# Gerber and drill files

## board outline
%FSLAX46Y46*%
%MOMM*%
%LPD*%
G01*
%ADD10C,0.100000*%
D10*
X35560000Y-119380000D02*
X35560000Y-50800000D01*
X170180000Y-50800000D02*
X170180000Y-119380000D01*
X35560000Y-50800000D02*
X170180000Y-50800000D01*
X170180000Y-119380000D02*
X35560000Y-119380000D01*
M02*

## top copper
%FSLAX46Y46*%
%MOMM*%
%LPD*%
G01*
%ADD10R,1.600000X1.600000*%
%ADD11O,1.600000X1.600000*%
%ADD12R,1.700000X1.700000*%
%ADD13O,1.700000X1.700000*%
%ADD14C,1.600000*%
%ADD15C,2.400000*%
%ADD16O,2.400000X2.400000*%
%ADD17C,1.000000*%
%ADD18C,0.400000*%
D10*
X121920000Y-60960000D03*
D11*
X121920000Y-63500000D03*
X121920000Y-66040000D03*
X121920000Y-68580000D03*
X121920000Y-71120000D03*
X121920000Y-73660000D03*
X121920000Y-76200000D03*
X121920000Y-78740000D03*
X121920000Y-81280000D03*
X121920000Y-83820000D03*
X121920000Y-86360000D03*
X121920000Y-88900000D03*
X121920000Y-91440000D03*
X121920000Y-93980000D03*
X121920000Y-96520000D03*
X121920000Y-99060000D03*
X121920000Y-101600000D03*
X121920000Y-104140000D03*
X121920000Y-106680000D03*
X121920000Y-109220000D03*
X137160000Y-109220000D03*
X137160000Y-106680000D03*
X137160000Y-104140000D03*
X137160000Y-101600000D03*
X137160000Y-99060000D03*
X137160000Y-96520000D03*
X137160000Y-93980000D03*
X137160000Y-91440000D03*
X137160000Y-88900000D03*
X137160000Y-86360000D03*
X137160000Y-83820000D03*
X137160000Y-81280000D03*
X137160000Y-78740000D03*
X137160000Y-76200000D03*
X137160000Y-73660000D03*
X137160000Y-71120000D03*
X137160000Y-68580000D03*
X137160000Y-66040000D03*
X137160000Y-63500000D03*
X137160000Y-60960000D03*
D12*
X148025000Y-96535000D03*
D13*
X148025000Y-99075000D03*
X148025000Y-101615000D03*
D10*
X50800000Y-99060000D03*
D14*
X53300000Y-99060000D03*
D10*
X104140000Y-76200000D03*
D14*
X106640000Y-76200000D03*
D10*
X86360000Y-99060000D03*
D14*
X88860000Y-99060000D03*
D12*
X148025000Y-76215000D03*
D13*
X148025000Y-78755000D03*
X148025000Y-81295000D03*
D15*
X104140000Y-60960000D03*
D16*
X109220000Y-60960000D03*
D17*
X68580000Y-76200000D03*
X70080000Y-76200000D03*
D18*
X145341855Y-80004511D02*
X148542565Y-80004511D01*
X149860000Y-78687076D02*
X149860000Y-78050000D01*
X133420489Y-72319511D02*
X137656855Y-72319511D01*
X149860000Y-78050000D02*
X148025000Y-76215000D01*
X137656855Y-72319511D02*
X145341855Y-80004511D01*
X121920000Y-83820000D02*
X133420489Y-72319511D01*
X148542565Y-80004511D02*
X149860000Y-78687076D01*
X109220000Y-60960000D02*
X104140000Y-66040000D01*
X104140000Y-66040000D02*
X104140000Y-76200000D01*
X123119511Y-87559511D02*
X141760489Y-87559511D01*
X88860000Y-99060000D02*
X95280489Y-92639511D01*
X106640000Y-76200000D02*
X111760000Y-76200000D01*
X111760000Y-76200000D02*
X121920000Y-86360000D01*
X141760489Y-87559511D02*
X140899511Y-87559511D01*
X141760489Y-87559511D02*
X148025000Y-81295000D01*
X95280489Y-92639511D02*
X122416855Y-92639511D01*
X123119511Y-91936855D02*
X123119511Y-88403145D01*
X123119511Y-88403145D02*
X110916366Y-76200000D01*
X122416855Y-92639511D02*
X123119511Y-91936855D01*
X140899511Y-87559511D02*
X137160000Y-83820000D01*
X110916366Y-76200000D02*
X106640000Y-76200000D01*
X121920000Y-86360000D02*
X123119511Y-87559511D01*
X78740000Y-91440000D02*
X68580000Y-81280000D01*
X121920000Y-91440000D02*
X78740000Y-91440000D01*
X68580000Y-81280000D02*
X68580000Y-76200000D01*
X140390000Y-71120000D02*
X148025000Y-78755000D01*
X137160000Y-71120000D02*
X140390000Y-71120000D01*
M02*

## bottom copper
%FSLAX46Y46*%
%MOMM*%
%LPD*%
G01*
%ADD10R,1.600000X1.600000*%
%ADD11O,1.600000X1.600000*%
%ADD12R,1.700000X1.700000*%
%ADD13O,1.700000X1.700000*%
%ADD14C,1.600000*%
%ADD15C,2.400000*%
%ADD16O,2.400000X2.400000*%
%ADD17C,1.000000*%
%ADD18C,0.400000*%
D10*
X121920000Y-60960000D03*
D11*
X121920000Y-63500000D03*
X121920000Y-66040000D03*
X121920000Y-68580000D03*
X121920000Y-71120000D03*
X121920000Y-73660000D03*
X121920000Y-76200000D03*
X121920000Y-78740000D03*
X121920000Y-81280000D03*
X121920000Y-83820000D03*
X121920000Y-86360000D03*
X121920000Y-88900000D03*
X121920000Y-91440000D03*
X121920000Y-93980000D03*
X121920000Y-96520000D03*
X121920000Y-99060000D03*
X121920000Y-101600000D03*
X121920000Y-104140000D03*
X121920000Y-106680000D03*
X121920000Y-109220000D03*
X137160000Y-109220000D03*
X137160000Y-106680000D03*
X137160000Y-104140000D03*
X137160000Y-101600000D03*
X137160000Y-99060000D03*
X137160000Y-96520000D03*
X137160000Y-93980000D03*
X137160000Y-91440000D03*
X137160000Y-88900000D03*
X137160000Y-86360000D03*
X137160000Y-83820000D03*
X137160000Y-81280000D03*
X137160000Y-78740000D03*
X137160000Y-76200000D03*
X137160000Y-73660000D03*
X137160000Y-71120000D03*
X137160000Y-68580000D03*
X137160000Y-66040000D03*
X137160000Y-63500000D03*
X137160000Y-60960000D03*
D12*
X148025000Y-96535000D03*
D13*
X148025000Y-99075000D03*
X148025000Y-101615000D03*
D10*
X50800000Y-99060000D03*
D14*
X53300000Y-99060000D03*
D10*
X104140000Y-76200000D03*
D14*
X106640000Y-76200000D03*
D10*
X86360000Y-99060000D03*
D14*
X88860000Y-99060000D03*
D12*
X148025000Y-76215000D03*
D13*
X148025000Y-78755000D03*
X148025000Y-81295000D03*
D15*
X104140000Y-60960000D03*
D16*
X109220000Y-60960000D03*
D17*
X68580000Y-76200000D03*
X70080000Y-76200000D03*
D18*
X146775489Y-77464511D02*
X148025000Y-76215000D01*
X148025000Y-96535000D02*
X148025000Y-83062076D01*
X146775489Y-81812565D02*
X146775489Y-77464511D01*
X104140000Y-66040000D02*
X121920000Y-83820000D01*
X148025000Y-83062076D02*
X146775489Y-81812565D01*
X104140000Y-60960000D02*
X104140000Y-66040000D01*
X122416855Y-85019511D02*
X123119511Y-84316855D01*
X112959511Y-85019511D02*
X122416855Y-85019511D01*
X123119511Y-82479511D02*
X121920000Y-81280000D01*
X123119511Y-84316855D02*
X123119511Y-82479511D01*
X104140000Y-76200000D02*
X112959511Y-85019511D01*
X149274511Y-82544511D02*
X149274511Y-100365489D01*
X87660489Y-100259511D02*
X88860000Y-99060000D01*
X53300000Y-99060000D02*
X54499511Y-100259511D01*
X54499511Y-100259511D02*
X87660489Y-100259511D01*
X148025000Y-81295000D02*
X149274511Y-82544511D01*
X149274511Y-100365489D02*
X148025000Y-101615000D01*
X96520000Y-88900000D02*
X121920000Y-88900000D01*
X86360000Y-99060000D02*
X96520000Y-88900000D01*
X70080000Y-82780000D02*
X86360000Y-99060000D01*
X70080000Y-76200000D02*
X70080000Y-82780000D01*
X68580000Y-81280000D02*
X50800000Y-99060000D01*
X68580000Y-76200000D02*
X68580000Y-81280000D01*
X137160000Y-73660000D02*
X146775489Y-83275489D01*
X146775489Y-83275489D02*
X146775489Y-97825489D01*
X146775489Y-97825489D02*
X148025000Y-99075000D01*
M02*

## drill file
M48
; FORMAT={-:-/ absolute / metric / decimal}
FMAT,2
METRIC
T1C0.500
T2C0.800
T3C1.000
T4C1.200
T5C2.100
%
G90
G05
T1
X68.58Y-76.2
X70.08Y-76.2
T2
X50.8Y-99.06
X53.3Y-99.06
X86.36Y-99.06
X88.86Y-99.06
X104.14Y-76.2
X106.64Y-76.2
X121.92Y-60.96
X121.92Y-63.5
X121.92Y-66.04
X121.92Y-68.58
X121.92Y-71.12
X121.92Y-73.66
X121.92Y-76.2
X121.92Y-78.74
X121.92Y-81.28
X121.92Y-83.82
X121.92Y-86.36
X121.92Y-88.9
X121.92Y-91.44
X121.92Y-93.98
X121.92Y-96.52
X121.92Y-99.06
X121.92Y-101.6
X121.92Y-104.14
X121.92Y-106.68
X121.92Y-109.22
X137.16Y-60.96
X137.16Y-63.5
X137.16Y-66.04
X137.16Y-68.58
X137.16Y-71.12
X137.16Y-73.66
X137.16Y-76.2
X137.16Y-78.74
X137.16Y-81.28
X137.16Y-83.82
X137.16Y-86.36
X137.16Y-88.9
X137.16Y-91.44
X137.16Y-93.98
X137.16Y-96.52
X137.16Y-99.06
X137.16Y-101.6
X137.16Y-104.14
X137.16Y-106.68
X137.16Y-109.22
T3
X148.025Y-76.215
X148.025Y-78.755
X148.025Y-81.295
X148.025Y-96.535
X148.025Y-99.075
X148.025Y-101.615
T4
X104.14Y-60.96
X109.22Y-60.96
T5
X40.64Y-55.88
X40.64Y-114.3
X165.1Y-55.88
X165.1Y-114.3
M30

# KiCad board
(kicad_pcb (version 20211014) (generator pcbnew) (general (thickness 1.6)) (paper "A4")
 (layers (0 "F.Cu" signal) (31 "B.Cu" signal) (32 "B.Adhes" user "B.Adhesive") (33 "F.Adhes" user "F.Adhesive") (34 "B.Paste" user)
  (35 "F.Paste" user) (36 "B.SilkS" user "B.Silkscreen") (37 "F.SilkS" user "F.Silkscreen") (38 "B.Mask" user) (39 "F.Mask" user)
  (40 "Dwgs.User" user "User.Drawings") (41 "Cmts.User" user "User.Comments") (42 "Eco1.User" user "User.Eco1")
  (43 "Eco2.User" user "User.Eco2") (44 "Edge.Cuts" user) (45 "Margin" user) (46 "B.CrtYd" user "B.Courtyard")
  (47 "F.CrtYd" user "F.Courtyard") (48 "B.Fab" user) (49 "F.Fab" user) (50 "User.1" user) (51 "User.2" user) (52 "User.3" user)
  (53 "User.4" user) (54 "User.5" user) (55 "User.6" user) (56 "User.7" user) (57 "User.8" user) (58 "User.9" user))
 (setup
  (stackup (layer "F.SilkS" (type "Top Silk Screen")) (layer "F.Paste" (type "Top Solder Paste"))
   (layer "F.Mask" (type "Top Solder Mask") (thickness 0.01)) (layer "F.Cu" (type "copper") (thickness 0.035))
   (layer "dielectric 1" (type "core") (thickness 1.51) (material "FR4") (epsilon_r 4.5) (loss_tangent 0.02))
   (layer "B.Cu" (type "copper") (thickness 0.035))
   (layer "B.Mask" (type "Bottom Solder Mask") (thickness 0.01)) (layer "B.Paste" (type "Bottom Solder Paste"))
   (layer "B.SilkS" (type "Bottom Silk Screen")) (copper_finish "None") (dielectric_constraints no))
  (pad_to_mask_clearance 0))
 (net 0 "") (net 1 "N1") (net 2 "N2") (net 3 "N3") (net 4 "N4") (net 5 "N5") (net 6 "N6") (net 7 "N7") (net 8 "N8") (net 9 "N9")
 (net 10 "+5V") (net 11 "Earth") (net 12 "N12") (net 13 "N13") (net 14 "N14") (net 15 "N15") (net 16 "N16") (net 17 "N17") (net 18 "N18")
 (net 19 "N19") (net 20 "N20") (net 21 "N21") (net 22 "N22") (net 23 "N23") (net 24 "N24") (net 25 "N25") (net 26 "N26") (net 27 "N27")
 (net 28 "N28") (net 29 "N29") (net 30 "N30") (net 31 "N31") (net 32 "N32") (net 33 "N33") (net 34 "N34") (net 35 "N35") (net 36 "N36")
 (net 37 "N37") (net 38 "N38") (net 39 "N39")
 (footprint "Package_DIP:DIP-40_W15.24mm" (layer "F.Cu") (at 121.92 60.96)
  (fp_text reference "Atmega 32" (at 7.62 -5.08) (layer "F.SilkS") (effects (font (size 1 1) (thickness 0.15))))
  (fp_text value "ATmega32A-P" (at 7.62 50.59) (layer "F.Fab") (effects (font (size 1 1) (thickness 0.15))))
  (pad "1" thru_hole rect (at 0 0) (size 1.6 1.6) (drill 0.8) (layers *.Cu *.Mask) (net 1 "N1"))
  (pad "2" thru_hole oval (at 0 2.54) (size 1.6 1.6) (drill 0.8) (layers *.Cu *.Mask) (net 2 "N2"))
  (pad "3" thru_hole oval (at 0 5.08) (size 1.6 1.6) (drill 0.8) (layers *.Cu *.Mask) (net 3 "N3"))
  (pad "4" thru_hole oval (at 0 7.62) (size 1.6 1.6) (drill 0.8) (layers *.Cu *.Mask) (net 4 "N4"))
  (pad "5" thru_hole oval (at 0 10.16) (size 1.6 1.6) (drill 0.8) (layers *.Cu *.Mask) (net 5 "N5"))
  (pad "6" thru_hole oval (at 0 12.7) (size 1.6 1.6) (drill 0.8) (layers *.Cu *.Mask) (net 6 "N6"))
  (pad "7" thru_hole oval (at 0 15.24) (size 1.6 1.6) (drill 0.8) (layers *.Cu *.Mask) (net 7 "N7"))
  (pad "8" thru_hole oval (at 0 17.78) (size 1.6 1.6) (drill 0.8) (layers *.Cu *.Mask) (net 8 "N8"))
  (pad "9" thru_hole oval (at 0 20.32) (size 1.6 1.6) (drill 0.8) (layers *.Cu *.Mask) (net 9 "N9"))
  (pad "10" thru_hole oval (at 0 22.86) (size 1.6 1.6) (drill 0.8) (layers *.Cu *.Mask) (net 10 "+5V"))
  (pad "11" thru_hole oval (at 0 25.4) (size 1.6 1.6) (drill 0.8) (layers *.Cu *.Mask) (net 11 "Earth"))
  (pad "12" thru_hole oval (at 0 27.94) (size 1.6 1.6) (drill 0.8) (layers *.Cu *.Mask) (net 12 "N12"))
  (pad "13" thru_hole oval (at 0 30.48) (size 1.6 1.6) (drill 0.8) (layers *.Cu *.Mask) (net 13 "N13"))
  (pad "14" thru_hole oval (at 0 33.02) (size 1.6 1.6) (drill 0.8) (layers *.Cu *.Mask) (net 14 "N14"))
  (pad "15" thru_hole oval (at 0 35.56) (size 1.6 1.6) (drill 0.8) (layers *.Cu *.Mask) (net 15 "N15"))
  (pad "16" thru_hole oval (at 0 38.1) (size 1.6 1.6) (drill 0.8) (layers *.Cu *.Mask) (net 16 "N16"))
  (pad "17" thru_hole oval (at 0 40.64) (size 1.6 1.6) (drill 0.8) (layers *.Cu *.Mask) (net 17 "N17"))
  (pad "18" thru_hole oval (at 0 43.18) (size 1.6 1.6) (drill 0.8) (layers *.Cu *.Mask) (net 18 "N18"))
  (pad "19" thru_hole oval (at 0 45.72) (size 1.6 1.6) (drill 0.8) (layers *.Cu *.Mask) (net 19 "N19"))
  (pad "20" thru_hole oval (at 0 48.26) (size 1.6 1.6) (drill 0.8) (layers *.Cu *.Mask) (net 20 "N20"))
  (pad "21" thru_hole oval (at 15.24 48.26) (size 1.6 1.6) (drill 0.8) (layers *.Cu *.Mask) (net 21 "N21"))
  (pad "22" thru_hole oval (at 15.24 45.72) (size 1.6 1.6) (drill 0.8) (layers *.Cu *.Mask) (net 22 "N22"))
  (pad "23" thru_hole oval (at 15.24 43.18) (size 1.6 1.6) (drill 0.8) (layers *.Cu *.Mask) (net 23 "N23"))
  (pad "24" thru_hole oval (at 15.24 40.64) (size 1.6 1.6) (drill 0.8) (layers *.Cu *.Mask) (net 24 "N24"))
  (pad "25" thru_hole oval (at 15.24 38.1) (size 1.6 1.6) (drill 0.8) (layers *.Cu *.Mask) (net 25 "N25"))
  (pad "26" thru_hole oval (at 15.24 35.56) (size 1.6 1.6) (drill 0.8) (layers *.Cu *.Mask) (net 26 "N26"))
  (pad "27" thru_hole oval (at 15.24 33.02) (size 1.6 1.6) (drill 0.8) (layers *.Cu *.Mask) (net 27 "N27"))
  (pad "28" thru_hole oval (at 15.24 30.48) (size 1.6 1.6) (drill 0.8) (layers *.Cu *.Mask) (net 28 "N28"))
  (pad "29" thru_hole oval (at 15.24 27.94) (size 1.6 1.6) (drill 0.8) (layers *.Cu *.Mask) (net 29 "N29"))
  (pad "30" thru_hole oval (at 15.24 25.4) (size 1.6 1.6) (drill 0.8) (layers *.Cu *.Mask) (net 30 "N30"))
  (pad "31" thru_hole oval (at 15.24 22.86) (size 1.6 1.6) (drill 0.8) (layers *.Cu *.Mask) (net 11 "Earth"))
  (pad "32" thru_hole oval (at 15.24 20.32) (size 1.6 1.6) (drill 0.8) (layers *.Cu *.Mask) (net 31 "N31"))
  (pad "33" thru_hole oval (at 15.24 17.78) (size 1.6 1.6) (drill 0.8) (layers *.Cu *.Mask) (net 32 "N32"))
  (pad "34" thru_hole oval (at 15.24 15.24) (size 1.6 1.6) (drill 0.8) (layers *.Cu *.Mask) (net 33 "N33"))
  (pad "35" thru_hole oval (at 15.24 12.7) (size 1.6 1.6) (drill 0.8) (layers *.Cu *.Mask) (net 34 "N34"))
  (pad "36" thru_hole oval (at 15.24 10.16) (size 1.6 1.6) (drill 0.8) (layers *.Cu *.Mask) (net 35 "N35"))
  (pad "37" thru_hole oval (at 15.24 7.62) (size 1.6 1.6) (drill 0.8) (layers *.Cu *.Mask) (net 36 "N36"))
  (pad "38" thru_hole oval (at 15.24 5.08) (size 1.6 1.6) (drill 0.8) (layers *.Cu *.Mask) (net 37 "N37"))
  (pad "39" thru_hole oval (at 15.24 2.54) (size 1.6 1.6) (drill 0.8) (layers *.Cu *.Mask) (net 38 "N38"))
  (pad "40" thru_hole oval (at 15.24 0) (size 1.6 1.6) (drill 0.8) (layers *.Cu *.Mask) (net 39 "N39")))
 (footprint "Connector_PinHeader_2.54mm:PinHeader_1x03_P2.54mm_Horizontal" (layer "F.Cu") (at 148.025 96.535)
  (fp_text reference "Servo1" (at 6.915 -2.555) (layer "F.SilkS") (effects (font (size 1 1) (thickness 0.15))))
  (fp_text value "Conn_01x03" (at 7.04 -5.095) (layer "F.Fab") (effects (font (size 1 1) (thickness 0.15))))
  (pad "1" thru_hole rect (at 0 0) (size 1.7 1.7) (drill 1) (layers *.Cu *.Mask) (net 10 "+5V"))
  (pad "2" thru_hole oval (at 0 2.54) (size 1.7 1.7) (drill 1) (layers *.Cu *.Mask) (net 34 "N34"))
  (pad "3" thru_hole oval (at 0 5.08) (size 1.7 1.7) (drill 1) (layers *.Cu *.Mask) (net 11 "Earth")))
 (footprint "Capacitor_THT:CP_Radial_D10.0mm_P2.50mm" (layer "F.Cu") (at 50.8 99.06)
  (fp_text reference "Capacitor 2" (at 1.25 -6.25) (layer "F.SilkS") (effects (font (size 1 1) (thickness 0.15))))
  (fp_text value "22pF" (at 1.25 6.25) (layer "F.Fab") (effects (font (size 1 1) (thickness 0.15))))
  (pad "1" thru_hole rect (at 0 0) (size 1.6 1.6) (drill 0.8) (layers *.Cu *.Mask) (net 13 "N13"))
  (pad "2" thru_hole circle (at 2.5 0) (size 1.6 1.6) (drill 0.8) (layers *.Cu *.Mask) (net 11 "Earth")))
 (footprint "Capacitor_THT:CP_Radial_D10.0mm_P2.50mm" (layer "F.Cu") (at 104.14 76.2)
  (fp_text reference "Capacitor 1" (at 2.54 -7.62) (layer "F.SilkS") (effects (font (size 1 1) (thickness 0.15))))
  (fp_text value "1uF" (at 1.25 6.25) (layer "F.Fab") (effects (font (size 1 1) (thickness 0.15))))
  (pad "1" thru_hole rect (at 0 0) (size 1.6 1.6) (drill 0.8) (layers *.Cu *.Mask) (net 9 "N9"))
  (pad "2" thru_hole circle (at 2.5 0) (size 1.6 1.6) (drill 0.8) (layers *.Cu *.Mask) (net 11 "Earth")))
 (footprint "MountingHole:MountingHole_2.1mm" (layer "F.Cu") (at 165.1 114.3)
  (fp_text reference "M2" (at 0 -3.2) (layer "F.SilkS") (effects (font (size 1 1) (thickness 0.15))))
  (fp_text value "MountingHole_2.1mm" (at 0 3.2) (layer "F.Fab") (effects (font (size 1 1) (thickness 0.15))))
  (pad "" np_thru_hole circle (at 0 0) (size 2.1 2.1) (drill 2.1) (layers *.Cu *.Mask)))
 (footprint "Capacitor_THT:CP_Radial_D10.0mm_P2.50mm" (layer "F.Cu") (at 86.36 99.06)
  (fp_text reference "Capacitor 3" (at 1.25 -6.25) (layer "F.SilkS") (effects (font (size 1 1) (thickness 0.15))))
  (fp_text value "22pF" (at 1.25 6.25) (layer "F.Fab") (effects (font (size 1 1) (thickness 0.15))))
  (pad "1" thru_hole rect (at 0 0) (size 1.6 1.6) (drill 0.8) (layers *.Cu *.Mask) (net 12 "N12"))
  (pad "2" thru_hole circle (at 2.5 0) (size 1.6 1.6) (drill 0.8) (layers *.Cu *.Mask) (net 11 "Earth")))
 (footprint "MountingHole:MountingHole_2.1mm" (layer "F.Cu") (at 40.64 55.88)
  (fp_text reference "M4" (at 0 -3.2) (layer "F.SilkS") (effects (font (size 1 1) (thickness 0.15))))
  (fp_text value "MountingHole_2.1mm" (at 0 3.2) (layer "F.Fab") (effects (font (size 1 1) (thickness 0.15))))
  (pad "" np_thru_hole circle (at 0 0) (size 2.1 2.1) (drill 2.1) (layers *.Cu *.Mask)))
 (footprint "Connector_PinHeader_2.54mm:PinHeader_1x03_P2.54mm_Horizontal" (layer "F.Cu") (at 148.025 76.215)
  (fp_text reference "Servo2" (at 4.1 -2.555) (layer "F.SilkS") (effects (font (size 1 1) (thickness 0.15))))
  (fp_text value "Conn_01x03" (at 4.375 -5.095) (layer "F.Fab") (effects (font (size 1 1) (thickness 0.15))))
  (pad "1" thru_hole rect (at 0 0) (size 1.7 1.7) (drill 1) (layers *.Cu *.Mask) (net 10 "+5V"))
  (pad "2" thru_hole oval (at 0 2.54) (size 1.7 1.7) (drill 1) (layers *.Cu *.Mask) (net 35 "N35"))
  (pad "3" thru_hole oval (at 0 5.08) (size 1.7 1.7) (drill 1) (layers *.Cu *.Mask) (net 11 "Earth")))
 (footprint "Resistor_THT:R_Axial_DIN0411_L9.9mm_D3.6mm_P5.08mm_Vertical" (layer "F.Cu") (at 104.14 60.96)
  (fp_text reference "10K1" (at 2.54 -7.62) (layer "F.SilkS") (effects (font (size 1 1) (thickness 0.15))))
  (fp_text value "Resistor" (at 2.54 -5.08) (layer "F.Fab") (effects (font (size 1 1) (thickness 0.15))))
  (pad "1" thru_hole circle (at 0 0) (size 2.4 2.4) (drill 1.2) (layers *.Cu *.Mask) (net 10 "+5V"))
  (pad "2" thru_hole oval (at 5.08 0) (size 2.4 2.4) (drill 1.2) (layers *.Cu *.Mask) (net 9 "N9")))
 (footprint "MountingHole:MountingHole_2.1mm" (layer "F.Cu") (at 40.64 114.3)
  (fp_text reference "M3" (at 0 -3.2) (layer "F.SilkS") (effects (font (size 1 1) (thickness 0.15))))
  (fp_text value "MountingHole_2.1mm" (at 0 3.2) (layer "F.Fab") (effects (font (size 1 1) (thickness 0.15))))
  (pad "" np_thru_hole circle (at 0 0) (size 2.1 2.1) (drill 2.1) (layers *.Cu *.Mask)))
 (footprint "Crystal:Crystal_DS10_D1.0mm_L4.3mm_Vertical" (layer "F.Cu") (at 68.58 76.2)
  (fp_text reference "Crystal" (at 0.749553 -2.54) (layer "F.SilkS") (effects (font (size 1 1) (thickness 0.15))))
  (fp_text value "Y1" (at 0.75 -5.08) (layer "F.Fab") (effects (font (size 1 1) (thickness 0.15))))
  (pad "1" thru_hole circle (at 0 0) (size 1 1) (drill 0.5) (layers *.Cu *.Mask) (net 13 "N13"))
  (pad "2" thru_hole circle (at 1.5 0) (size 1 1) (drill 0.5) (layers *.Cu *.Mask) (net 12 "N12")))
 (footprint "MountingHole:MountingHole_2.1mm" (layer "F.Cu") (at 165.1 55.88)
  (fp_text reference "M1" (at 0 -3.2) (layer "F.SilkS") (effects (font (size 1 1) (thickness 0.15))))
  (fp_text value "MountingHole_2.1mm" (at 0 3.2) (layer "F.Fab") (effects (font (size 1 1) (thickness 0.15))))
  (pad "" np_thru_hole circle (at 0 0) (size 2.1 2.1) (drill 2.1) (layers *.Cu *.Mask)))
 (gr_line (start 35.56 119.38) (end 35.56 50.8) (layer "Edge.Cuts") (width 0.1))
 (gr_line (start 170.18 50.8) (end 170.18 119.38) (layer "Edge.Cuts") (width 0.1))
 (gr_line (start 35.56 50.8) (end 170.18 50.8) (layer "Edge.Cuts") (width 0.1))
 (gr_line (start 170.18 119.38) (end 35.56 119.38) (layer "Edge.Cuts") (width 0.1))
 (segment (start 145.341855 80.004511) (end 148.542565 80.004511) (width 0.4) (layer "F.Cu") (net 10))
 (segment (start 149.86 78.687076) (end 149.86 78.05) (width 0.4) (layer "F.Cu") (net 10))
 (segment (start 133.420489 72.319511) (end 137.656855 72.319511) (width 0.4) (layer "F.Cu") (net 10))
 (segment (start 149.86 78.05) (end 148.025 76.215) (width 0.4) (layer "F.Cu") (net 10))
 (segment (start 137.656855 72.319511) (end 145.341855 80.004511) (width 0.4) (layer "F.Cu") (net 10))
 (segment (start 121.92 83.82) (end 133.420489 72.319511) (width 0.4) (layer "F.Cu") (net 10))
 (segment (start 148.542565 80.004511) (end 149.86 78.687076) (width 0.4) (layer "F.Cu") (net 10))
 (segment (start 146.775489 77.464511) (end 148.025 76.215) (width 0.4) (layer "B.Cu") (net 10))
 (segment (start 148.025 96.535) (end 148.025 83.062076) (width 0.4) (layer "B.Cu") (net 10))
 (segment (start 146.775489 81.812565) (end 146.775489 77.464511) (width 0.4) (layer "B.Cu") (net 10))
 (segment (start 104.14 66.04) (end 121.92 83.82) (width 0.4) (layer "B.Cu") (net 10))
 (segment (start 148.025 83.062076) (end 146.775489 81.812565) (width 0.4) (layer "B.Cu") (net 10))
 (segment (start 104.14 60.96) (end 104.14 66.04) (width 0.4) (layer "B.Cu") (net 10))
 (segment (start 109.22 60.96) (end 104.14 66.04) (width 0.4) (layer "F.Cu") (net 9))
 (segment (start 104.14 66.04) (end 104.14 76.2) (width 0.4) (layer "F.Cu") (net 9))
 (segment (start 122.416855 85.019511) (end 123.119511 84.316855) (width 0.4) (layer "B.Cu") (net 9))
 (segment (start 112.959511 85.019511) (end 122.416855 85.019511) (width 0.4) (layer "B.Cu") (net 9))
 (segment (start 123.119511 82.479511) (end 121.92 81.28) (width 0.4) (layer "B.Cu") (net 9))
 (segment (start 123.119511 84.316855) (end 123.119511 82.479511) (width 0.4) (layer "B.Cu") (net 9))
 (segment (start 104.14 76.2) (end 112.959511 85.019511) (width 0.4) (layer "B.Cu") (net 9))
 (segment (start 123.119511 87.559511) (end 141.760489 87.559511) (width 0.4) (layer "F.Cu") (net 11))
 (segment (start 88.86 99.06) (end 95.280489 92.639511) (width 0.4) (layer "F.Cu") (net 11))
 (segment (start 106.64 76.2) (end 111.76 76.2) (width 0.4) (layer "F.Cu") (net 11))
 (segment (start 111.76 76.2) (end 121.92 86.36) (width 0.4) (layer "F.Cu") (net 11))
 (segment (start 141.760489 87.559511) (end 140.899511 87.559511) (width 0.4) (layer "F.Cu") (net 11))
 (segment (start 141.760489 87.559511) (end 148.025 81.295) (width 0.4) (layer "F.Cu") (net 11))
 (segment (start 95.280489 92.639511) (end 122.416855 92.639511) (width 0.4) (layer "F.Cu") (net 11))
 (segment (start 123.119511 91.936855) (end 123.119511 88.403145) (width 0.4) (layer "F.Cu") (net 11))
 (segment (start 123.119511 88.403145) (end 110.916366 76.2) (width 0.4) (layer "F.Cu") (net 11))
 (segment (start 122.416855 92.639511) (end 123.119511 91.936855) (width 0.4) (layer "F.Cu") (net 11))
 (segment (start 140.899511 87.559511) (end 137.16 83.82) (width 0.4) (layer "F.Cu") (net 11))
 (segment (start 110.916366 76.2) (end 106.64 76.2) (width 0.4) (layer "F.Cu") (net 11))
 (segment (start 121.92 86.36) (end 123.119511 87.559511) (width 0.4) (layer "F.Cu") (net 11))
 (segment (start 149.274511 82.544511) (end 149.274511 100.365489) (width 0.4) (layer "B.Cu") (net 11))
 (segment (start 87.660489 100.259511) (end 88.86 99.06) (width 0.4) (layer "B.Cu") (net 11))
 (segment (start 53.3 99.06) (end 54.499511 100.259511) (width 0.4) (layer "B.Cu") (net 11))
 (segment (start 54.499511 100.259511) (end 87.660489 100.259511) (width 0.4) (layer "B.Cu") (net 11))
 (segment (start 148.025 81.295) (end 149.274511 82.544511) (width 0.4) (layer "B.Cu") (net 11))
 (segment (start 149.274511 100.365489) (end 148.025 101.615) (width 0.4) (layer "B.Cu") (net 11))
 (segment (start 96.52 88.9) (end 121.92 88.9) (width 0.4) (layer "B.Cu") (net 12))
 (segment (start 86.36 99.06) (end 96.52 88.9) (width 0.4) (layer "B.Cu") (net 12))
 (segment (start 70.08 82.78) (end 86.36 99.06) (width 0.4) (layer "B.Cu") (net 12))
 (segment (start 70.08 76.2) (end 70.08 82.78) (width 0.4) (layer "B.Cu") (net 12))
 (segment (start 78.74 91.44) (end 68.58 81.28) (width 0.4) (layer "F.Cu") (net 13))
 (segment (start 121.92 91.44) (end 78.74 91.44) (width 0.4) (layer "F.Cu") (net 13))
 (segment (start 68.58 81.28) (end 68.58 76.2) (width 0.4) (layer "F.Cu") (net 13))
 (segment (start 68.58 81.28) (end 50.8 99.06) (width 0.4) (layer "B.Cu") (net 13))
 (segment (start 68.58 76.2) (end 68.58 81.28) (width 0.4) (layer "B.Cu") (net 13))
 (segment (start 137.16 73.66) (end 146.775489 83.275489) (width 0.4) (layer "B.Cu") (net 34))
 (segment (start 146.775489 83.275489) (end 146.775489 97.825489) (width 0.4) (layer "B.Cu") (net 34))
 (segment (start 146.775489 97.825489) (end 148.025 99.075) (width 0.4) (layer "B.Cu") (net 34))
 (segment (start 140.39 71.12) (end 148.025 78.755) (width 0.4) (layer "F.Cu") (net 35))
 (segment (start 137.16 71.12) (end 140.39 71.12) (width 0.4) (layer "F.Cu") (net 35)))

